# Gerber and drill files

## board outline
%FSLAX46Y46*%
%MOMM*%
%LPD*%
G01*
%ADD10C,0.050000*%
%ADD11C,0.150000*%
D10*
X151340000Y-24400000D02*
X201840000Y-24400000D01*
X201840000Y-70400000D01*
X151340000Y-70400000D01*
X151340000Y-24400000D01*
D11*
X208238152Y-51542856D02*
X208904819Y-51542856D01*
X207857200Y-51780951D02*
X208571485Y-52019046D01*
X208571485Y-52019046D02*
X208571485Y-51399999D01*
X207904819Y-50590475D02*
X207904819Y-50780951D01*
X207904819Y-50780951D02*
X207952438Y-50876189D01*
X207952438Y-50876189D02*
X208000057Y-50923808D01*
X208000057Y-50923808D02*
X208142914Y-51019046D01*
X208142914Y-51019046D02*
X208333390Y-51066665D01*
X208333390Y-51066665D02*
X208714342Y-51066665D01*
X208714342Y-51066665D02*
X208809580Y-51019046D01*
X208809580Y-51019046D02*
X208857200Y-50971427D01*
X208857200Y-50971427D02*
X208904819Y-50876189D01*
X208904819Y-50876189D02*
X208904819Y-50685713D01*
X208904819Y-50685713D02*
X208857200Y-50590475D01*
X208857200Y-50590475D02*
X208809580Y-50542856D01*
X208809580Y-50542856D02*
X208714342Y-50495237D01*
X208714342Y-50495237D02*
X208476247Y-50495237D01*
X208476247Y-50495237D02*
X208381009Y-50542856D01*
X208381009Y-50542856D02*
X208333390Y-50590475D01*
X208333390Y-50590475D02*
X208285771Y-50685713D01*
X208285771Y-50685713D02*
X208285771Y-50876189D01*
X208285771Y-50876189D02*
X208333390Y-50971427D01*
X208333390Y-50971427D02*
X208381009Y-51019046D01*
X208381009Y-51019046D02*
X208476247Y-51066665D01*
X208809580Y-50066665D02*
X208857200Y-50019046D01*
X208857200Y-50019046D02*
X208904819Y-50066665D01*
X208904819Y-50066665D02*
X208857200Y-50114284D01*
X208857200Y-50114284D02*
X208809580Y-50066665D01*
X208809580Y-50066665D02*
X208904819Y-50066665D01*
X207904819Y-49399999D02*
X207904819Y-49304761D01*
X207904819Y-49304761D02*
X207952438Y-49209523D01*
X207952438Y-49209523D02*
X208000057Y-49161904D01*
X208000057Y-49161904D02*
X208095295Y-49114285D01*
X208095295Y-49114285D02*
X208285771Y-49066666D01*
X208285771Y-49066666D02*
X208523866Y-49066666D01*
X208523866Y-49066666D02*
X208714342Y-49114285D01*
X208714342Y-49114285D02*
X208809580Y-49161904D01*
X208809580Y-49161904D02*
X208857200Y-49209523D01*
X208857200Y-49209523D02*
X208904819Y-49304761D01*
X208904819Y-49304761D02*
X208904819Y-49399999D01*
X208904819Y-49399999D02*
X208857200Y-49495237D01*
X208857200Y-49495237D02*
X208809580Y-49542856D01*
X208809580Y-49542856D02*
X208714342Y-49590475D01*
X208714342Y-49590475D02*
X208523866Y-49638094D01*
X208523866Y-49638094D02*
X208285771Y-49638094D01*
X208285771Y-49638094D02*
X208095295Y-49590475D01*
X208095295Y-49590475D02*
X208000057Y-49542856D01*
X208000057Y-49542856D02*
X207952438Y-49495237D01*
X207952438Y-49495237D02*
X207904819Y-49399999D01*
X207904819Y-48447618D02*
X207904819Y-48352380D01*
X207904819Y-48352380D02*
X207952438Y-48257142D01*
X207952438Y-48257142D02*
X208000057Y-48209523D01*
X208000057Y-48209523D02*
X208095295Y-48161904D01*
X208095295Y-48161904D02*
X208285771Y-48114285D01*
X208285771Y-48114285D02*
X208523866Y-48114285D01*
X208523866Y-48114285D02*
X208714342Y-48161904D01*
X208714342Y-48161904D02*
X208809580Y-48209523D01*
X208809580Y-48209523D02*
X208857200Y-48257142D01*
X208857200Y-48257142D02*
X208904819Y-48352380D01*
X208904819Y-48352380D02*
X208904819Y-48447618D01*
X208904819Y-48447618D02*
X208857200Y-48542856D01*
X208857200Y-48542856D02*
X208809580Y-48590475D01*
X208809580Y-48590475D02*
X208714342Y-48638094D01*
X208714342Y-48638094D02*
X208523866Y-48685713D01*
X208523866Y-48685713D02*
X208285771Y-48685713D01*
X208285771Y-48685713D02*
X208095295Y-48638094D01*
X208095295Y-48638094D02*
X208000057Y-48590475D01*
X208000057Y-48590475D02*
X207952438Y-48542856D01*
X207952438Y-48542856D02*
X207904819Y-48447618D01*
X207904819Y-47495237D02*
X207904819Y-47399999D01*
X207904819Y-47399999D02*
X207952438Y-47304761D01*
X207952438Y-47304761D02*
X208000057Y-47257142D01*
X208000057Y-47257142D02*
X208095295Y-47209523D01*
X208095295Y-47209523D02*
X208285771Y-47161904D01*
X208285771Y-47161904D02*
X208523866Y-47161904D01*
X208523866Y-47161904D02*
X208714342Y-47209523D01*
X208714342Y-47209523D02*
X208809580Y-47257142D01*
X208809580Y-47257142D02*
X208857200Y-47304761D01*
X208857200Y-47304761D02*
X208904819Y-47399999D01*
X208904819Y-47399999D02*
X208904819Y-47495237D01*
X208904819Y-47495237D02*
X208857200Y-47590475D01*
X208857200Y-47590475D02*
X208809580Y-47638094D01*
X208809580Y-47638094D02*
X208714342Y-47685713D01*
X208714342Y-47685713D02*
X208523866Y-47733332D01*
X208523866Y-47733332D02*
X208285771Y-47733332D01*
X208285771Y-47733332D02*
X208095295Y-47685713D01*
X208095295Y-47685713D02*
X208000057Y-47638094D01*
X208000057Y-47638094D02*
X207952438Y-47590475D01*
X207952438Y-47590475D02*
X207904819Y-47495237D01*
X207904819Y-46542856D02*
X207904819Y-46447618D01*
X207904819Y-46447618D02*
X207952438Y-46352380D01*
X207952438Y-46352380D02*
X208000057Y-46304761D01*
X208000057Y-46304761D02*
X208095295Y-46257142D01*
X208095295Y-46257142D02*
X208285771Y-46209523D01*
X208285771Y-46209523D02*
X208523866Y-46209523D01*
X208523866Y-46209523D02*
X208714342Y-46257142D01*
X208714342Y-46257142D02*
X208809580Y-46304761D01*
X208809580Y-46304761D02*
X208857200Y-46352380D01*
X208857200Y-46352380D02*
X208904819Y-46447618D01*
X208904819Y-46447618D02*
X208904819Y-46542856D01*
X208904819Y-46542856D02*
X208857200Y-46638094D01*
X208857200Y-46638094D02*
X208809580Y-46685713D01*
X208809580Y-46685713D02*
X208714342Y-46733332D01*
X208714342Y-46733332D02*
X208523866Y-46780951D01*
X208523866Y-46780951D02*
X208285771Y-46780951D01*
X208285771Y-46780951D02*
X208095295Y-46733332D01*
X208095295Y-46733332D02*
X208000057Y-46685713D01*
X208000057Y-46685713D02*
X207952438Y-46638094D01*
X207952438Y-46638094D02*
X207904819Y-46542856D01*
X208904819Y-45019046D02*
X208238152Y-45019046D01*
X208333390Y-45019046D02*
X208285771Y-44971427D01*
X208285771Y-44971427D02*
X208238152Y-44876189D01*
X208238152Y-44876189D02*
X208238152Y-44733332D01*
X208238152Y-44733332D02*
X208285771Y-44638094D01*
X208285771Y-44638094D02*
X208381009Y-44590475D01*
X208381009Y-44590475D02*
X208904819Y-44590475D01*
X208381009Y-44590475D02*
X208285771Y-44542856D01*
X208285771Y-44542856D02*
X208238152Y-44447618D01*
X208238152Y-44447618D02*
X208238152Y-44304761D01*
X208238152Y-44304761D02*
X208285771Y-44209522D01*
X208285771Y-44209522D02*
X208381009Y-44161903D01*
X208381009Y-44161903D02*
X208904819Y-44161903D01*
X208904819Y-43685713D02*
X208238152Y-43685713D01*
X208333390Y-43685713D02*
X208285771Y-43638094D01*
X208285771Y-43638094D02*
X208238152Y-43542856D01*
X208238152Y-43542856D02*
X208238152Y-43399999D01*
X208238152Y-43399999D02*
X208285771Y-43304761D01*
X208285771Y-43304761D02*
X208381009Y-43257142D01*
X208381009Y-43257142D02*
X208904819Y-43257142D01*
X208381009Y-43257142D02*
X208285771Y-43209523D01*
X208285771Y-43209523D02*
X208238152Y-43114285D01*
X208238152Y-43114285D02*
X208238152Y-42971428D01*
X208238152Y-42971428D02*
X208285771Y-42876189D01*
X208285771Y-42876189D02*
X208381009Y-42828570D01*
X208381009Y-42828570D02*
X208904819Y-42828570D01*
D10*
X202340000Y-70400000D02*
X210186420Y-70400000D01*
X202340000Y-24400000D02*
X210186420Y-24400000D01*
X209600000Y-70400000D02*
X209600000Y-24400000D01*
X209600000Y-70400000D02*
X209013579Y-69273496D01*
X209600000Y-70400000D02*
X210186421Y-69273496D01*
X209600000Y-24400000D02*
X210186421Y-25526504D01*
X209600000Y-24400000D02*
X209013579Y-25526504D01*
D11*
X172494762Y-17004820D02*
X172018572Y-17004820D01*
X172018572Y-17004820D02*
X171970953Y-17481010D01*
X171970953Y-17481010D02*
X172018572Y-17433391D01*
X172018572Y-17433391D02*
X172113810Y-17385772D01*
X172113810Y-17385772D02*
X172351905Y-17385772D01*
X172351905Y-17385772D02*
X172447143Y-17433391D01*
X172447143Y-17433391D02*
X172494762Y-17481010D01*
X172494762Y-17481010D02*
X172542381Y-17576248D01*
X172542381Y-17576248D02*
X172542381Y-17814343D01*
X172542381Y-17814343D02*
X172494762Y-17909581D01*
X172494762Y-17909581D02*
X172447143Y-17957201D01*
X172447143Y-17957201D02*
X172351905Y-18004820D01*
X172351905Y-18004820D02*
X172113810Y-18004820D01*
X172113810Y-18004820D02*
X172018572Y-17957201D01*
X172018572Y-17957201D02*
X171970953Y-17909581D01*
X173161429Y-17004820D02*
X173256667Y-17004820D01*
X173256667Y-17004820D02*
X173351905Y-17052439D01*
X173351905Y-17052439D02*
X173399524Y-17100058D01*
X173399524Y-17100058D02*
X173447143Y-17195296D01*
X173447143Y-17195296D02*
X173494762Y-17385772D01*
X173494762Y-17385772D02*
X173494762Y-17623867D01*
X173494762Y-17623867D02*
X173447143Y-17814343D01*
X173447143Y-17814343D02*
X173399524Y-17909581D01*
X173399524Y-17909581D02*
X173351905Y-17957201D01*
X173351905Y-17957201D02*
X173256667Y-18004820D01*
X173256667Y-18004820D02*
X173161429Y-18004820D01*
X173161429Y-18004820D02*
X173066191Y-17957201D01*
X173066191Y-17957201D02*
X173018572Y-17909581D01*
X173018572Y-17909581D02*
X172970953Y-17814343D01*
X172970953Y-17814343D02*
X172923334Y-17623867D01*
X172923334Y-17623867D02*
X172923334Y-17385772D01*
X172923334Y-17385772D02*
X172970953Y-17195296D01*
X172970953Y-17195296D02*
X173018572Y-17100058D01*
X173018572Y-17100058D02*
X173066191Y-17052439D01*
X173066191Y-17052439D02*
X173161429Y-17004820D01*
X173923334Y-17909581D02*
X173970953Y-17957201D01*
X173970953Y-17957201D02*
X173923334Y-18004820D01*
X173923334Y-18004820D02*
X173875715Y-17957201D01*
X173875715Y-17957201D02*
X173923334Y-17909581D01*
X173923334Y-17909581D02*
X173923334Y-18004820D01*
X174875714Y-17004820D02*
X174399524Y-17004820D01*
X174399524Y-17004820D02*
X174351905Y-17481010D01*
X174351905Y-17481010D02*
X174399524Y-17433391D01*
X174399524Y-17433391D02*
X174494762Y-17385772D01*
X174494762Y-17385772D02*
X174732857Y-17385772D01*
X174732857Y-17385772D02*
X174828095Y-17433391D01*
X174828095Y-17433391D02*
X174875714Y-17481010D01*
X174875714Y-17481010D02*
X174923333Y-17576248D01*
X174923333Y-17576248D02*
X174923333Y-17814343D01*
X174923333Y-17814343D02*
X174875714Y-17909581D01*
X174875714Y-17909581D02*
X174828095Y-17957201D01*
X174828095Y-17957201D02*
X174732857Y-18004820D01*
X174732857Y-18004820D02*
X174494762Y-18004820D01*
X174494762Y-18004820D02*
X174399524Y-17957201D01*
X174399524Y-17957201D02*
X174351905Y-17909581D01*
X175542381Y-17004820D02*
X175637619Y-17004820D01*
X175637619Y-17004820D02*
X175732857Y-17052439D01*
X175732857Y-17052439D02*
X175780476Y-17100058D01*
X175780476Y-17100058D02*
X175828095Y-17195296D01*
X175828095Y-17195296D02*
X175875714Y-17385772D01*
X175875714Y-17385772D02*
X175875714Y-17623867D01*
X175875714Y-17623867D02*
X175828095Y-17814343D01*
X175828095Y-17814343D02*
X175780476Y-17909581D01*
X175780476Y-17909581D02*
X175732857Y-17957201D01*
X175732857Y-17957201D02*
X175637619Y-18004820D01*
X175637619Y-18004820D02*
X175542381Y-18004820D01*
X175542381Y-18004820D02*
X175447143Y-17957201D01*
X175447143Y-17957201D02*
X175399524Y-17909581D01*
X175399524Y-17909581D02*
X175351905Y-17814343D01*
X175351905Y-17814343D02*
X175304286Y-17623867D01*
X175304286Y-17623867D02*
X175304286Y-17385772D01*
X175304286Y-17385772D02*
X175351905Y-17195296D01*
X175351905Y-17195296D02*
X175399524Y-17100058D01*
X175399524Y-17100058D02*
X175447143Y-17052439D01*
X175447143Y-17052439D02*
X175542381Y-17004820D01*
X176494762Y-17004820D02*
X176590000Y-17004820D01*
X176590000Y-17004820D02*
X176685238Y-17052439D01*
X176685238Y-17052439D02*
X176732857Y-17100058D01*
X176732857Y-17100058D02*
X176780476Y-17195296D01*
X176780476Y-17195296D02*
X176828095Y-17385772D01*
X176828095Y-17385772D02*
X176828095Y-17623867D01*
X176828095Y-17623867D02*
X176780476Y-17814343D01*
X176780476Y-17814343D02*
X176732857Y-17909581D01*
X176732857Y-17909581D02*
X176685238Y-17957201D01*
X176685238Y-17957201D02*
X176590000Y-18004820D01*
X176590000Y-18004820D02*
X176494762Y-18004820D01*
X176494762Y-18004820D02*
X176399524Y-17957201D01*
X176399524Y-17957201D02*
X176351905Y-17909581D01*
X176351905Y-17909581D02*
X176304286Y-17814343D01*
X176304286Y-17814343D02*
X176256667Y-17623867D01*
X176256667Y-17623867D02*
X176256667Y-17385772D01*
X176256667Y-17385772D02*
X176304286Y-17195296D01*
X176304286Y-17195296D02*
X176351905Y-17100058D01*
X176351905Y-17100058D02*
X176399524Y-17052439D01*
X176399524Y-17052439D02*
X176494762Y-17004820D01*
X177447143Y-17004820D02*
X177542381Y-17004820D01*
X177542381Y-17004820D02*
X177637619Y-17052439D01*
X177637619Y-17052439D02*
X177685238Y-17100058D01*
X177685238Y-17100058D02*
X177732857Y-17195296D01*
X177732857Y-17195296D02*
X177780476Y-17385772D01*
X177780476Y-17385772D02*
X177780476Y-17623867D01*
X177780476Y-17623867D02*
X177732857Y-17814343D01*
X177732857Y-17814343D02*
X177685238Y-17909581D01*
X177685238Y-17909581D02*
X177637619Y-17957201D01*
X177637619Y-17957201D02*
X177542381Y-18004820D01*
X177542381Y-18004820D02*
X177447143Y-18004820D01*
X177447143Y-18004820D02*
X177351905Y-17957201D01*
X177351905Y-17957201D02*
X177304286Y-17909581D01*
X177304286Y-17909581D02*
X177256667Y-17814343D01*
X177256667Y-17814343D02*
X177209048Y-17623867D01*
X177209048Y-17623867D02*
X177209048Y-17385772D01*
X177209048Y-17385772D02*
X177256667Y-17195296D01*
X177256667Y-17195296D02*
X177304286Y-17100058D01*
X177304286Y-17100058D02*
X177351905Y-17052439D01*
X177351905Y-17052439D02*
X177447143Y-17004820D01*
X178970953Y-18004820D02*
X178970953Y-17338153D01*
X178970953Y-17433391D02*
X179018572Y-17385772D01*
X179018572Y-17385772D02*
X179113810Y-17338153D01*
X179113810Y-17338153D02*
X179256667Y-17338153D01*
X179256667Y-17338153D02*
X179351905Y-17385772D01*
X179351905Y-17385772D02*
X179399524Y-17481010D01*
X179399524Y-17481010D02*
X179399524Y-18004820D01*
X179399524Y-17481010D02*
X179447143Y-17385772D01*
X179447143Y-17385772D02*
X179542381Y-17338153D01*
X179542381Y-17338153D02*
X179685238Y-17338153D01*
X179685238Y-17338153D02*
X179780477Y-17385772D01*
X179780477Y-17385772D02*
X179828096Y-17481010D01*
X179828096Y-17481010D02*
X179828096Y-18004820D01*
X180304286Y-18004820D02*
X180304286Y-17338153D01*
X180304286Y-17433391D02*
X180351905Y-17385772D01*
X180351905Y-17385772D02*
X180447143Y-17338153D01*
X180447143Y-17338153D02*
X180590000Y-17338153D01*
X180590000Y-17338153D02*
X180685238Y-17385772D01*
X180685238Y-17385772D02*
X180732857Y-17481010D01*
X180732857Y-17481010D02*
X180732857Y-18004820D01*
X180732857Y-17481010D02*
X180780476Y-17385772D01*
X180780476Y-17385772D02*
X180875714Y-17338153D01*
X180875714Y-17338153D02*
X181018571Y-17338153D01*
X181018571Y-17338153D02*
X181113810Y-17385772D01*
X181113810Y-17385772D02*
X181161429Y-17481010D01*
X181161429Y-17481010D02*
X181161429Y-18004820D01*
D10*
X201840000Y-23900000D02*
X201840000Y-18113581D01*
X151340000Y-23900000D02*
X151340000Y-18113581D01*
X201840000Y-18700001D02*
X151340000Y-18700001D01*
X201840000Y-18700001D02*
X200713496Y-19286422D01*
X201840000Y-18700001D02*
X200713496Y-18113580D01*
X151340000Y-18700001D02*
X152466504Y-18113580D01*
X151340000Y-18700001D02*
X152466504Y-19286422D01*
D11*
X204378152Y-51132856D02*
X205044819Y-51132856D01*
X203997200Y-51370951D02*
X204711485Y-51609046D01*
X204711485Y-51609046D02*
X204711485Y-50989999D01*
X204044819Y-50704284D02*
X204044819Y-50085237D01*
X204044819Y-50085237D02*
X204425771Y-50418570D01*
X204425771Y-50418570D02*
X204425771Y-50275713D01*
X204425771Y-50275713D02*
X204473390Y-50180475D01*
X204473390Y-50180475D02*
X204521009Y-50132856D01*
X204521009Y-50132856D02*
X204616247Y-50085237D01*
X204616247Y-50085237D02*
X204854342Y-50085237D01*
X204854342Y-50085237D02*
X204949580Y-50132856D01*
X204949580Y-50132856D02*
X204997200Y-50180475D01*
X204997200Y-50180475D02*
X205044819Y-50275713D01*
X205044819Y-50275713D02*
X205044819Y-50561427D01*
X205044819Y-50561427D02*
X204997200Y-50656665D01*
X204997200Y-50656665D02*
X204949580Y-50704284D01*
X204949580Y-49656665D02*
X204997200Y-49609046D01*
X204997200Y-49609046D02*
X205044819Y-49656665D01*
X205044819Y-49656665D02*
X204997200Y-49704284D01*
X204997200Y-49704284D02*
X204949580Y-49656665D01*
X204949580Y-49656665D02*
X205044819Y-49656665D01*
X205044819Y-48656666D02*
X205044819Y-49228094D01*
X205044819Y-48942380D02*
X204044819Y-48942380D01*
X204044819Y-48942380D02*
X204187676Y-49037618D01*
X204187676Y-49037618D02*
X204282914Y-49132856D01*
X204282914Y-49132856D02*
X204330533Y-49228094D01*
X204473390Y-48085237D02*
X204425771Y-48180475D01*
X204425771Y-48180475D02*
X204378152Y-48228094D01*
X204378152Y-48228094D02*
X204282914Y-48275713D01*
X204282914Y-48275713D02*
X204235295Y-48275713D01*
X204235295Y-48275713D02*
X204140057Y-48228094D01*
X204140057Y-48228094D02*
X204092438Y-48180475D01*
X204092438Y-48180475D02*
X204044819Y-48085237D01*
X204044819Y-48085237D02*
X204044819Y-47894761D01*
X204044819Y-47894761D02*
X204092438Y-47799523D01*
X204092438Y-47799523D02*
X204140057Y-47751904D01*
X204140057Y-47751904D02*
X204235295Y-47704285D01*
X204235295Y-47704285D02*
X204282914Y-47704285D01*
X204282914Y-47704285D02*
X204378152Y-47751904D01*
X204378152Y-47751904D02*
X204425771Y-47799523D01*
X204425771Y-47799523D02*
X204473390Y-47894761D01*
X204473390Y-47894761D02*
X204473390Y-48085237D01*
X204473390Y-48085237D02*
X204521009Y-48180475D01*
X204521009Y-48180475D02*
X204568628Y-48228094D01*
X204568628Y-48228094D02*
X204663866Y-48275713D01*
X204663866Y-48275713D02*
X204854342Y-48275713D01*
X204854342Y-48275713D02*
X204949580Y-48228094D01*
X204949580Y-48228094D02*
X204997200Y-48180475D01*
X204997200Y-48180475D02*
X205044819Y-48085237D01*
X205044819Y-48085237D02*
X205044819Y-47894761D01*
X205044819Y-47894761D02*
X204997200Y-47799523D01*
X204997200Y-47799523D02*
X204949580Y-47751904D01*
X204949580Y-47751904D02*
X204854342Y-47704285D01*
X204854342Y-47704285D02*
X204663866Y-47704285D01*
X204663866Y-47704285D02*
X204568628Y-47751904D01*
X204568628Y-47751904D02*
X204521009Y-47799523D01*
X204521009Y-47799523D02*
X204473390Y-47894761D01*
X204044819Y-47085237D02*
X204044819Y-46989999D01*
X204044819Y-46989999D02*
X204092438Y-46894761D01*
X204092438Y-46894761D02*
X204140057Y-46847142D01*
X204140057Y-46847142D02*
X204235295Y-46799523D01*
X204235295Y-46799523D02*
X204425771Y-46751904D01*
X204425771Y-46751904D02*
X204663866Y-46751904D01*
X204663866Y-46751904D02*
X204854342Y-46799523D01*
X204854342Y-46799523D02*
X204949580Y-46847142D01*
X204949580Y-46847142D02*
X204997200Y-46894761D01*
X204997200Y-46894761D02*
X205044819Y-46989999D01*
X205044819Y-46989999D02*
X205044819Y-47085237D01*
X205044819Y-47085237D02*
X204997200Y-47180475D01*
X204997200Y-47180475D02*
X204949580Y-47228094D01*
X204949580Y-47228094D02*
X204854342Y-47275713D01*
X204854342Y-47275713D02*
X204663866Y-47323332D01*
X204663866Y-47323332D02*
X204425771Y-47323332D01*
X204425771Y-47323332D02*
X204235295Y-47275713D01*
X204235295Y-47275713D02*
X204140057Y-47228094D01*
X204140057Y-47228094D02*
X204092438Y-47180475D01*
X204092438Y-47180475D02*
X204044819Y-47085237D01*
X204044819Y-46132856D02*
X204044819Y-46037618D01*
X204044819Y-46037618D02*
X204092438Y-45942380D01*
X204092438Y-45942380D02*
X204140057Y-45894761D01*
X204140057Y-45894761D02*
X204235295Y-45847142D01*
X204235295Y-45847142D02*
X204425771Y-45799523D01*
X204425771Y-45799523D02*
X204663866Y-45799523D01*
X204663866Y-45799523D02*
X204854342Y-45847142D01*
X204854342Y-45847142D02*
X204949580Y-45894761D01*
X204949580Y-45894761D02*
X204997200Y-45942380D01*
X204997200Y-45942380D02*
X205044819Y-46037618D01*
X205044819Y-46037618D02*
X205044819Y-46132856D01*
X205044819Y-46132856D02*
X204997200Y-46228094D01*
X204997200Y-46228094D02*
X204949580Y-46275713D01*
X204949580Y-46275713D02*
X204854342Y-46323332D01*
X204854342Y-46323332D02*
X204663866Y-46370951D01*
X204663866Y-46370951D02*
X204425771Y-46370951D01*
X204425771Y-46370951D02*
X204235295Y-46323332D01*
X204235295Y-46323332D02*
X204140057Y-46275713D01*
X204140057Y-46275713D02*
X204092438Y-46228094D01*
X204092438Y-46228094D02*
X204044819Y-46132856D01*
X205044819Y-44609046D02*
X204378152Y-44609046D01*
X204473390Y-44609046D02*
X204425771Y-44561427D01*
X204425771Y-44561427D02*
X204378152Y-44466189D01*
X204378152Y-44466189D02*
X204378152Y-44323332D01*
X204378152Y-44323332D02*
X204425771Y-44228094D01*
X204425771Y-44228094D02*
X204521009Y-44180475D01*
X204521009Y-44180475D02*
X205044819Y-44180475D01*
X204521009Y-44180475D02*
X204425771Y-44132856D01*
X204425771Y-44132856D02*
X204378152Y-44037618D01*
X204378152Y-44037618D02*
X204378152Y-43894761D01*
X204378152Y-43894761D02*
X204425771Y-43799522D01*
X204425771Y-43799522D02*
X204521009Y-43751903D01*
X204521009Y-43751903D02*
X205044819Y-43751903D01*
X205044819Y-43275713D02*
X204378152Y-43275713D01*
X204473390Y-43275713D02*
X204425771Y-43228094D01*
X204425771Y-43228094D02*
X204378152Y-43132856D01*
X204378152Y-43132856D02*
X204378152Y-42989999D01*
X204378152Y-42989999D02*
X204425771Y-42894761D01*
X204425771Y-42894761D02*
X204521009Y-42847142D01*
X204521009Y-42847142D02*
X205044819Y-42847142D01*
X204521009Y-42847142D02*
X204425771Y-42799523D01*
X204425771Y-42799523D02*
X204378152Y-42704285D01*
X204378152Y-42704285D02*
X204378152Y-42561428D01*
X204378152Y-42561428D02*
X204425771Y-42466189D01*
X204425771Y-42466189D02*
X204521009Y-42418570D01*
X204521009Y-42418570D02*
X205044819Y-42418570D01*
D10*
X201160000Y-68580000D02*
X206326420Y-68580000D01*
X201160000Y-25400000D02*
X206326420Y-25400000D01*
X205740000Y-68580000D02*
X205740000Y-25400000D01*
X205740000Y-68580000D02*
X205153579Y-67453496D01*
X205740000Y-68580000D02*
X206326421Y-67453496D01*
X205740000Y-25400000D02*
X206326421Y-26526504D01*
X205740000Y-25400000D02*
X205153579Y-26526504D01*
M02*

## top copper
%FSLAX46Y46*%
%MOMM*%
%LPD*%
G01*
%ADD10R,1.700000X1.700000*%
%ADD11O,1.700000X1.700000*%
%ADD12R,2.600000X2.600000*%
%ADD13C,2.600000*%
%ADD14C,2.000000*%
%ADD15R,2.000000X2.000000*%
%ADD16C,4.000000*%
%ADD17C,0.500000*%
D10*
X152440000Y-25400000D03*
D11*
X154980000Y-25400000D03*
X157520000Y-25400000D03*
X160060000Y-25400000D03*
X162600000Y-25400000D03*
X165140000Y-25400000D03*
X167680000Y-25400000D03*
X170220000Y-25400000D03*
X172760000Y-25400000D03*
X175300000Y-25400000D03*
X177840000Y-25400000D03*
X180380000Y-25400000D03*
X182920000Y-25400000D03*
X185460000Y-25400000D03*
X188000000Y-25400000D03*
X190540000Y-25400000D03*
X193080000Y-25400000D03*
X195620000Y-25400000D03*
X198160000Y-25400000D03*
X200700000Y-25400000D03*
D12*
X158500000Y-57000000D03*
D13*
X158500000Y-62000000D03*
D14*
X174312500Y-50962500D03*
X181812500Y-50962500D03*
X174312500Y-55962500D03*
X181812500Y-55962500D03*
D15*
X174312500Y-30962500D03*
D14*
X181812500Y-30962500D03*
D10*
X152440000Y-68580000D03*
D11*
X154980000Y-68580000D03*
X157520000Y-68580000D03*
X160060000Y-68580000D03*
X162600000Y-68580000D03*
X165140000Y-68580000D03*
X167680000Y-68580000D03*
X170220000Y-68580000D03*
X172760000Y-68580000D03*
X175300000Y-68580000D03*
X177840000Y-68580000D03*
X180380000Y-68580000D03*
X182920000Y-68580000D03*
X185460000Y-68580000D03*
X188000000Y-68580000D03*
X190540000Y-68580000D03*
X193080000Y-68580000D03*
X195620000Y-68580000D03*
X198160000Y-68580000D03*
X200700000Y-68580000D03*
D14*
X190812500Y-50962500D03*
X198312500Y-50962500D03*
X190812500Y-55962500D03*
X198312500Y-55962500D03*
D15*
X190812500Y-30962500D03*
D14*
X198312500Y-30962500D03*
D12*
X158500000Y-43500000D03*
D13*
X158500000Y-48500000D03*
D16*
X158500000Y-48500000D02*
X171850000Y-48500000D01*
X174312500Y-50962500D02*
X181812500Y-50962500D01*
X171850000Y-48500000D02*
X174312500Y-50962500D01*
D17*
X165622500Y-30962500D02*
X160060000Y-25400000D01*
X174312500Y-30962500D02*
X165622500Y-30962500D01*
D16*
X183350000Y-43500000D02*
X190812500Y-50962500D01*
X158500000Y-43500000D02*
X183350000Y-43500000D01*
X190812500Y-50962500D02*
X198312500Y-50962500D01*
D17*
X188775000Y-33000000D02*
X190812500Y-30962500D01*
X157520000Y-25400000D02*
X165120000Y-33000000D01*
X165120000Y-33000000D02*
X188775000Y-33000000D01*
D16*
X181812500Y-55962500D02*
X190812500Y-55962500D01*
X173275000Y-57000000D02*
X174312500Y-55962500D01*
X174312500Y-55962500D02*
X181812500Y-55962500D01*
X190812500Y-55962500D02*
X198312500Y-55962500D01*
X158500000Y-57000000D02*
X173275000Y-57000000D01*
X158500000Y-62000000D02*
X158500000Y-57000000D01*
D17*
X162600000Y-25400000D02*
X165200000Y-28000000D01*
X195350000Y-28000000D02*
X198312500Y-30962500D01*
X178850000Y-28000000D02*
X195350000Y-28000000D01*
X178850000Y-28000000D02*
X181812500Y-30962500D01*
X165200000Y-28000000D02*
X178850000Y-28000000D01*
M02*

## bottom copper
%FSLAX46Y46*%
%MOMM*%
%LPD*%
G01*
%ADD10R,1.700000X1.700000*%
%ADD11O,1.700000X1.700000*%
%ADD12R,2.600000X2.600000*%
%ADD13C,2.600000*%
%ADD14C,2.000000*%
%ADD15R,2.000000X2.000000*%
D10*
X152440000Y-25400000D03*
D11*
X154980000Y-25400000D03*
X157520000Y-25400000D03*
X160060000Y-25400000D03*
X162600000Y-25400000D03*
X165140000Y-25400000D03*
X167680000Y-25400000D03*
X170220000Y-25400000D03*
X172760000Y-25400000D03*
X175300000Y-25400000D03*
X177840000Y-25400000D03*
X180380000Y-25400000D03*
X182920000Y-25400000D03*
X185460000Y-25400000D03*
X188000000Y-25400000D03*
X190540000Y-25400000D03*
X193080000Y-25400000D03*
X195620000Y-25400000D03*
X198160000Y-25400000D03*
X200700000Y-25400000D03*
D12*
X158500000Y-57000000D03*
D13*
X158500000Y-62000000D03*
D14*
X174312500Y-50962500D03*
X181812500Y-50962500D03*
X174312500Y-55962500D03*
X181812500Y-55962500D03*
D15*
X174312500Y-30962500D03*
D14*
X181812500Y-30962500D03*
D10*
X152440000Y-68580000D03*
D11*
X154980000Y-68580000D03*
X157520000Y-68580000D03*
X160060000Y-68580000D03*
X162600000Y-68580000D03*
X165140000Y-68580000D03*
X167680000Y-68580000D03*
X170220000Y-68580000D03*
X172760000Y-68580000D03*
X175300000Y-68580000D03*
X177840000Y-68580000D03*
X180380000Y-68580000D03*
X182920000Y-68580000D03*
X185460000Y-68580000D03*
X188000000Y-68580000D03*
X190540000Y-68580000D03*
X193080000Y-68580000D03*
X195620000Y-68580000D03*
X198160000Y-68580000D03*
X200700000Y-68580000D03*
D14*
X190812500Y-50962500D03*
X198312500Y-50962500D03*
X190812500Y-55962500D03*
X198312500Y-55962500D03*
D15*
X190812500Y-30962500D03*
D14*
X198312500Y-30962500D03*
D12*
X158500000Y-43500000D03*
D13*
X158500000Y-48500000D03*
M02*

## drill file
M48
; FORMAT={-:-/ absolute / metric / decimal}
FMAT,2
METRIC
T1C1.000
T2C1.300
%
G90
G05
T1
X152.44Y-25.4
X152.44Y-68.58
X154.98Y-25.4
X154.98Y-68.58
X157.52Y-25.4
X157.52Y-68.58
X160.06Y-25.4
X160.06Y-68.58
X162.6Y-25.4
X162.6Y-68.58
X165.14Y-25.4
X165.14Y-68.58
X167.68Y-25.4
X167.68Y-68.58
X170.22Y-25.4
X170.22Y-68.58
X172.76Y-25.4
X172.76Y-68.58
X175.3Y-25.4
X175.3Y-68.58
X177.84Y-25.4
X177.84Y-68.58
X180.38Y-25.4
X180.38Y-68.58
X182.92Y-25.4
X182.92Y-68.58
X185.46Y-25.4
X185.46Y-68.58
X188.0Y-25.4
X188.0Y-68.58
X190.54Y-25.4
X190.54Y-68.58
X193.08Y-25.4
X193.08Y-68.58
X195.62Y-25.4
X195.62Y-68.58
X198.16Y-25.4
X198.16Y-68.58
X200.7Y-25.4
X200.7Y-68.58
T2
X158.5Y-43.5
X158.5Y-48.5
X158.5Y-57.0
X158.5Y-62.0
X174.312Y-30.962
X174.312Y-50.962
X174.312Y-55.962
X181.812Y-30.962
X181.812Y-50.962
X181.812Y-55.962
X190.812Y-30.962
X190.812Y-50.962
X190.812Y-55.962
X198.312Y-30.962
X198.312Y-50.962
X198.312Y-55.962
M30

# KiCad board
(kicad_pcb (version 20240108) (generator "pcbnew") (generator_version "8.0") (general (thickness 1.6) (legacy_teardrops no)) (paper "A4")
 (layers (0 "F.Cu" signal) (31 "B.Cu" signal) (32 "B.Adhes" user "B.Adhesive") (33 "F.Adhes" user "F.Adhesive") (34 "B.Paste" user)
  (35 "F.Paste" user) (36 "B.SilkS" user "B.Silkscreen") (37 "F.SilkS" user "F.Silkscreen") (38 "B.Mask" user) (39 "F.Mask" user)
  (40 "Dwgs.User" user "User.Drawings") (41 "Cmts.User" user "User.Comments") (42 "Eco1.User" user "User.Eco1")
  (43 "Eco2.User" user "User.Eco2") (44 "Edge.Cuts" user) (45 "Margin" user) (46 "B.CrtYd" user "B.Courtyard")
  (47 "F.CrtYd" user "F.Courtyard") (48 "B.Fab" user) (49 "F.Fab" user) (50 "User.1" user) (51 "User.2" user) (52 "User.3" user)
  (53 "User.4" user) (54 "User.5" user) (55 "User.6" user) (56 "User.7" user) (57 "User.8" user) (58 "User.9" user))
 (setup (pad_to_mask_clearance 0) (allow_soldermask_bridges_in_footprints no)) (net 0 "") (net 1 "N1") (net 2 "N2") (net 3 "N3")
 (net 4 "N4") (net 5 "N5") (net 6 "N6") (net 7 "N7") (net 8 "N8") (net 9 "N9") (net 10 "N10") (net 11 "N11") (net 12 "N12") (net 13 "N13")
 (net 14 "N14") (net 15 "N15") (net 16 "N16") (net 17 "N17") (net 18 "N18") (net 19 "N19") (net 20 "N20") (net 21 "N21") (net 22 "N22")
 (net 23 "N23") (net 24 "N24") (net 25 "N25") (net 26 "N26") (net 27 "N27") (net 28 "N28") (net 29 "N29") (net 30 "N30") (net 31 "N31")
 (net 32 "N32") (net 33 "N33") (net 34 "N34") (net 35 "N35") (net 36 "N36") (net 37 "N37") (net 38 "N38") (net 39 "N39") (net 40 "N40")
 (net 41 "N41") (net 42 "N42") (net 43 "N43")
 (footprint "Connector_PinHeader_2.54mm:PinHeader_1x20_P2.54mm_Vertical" (layer "F.Cu") (at 152.44 25.4 90)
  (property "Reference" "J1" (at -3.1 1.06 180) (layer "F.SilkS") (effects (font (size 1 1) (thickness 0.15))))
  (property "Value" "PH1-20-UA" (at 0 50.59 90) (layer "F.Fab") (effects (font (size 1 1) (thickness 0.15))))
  (pad "1" thru_hole rect (at 0 0 90) (size 1.7 1.7) (drill 1) (layers "*.Cu" "*.Mask") (remove_unused_layers no) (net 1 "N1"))
  (pad "2" thru_hole oval (at 0 2.54 90) (size 1.7 1.7) (drill 1) (layers "*.Cu" "*.Mask") (remove_unused_layers no) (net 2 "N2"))
  (pad "3" thru_hole oval (at 0 5.08 90) (size 1.7 1.7) (drill 1) (layers "*.Cu" "*.Mask") (remove_unused_layers no) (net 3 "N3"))
  (pad "4" thru_hole oval (at 0 7.62 90) (size 1.7 1.7) (drill 1) (layers "*.Cu" "*.Mask") (remove_unused_layers no) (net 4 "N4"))
  (pad "5" thru_hole oval (at 0 10.16 90) (size 1.7 1.7) (drill 1) (layers "*.Cu" "*.Mask") (remove_unused_layers no) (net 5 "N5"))
  (pad "6" thru_hole oval (at 0 12.7 90) (size 1.7 1.7) (drill 1) (layers "*.Cu" "*.Mask") (remove_unused_layers no) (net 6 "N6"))
  (pad "7" thru_hole oval (at 0 15.24 90) (size 1.7 1.7) (drill 1) (layers "*.Cu" "*.Mask") (remove_unused_layers no) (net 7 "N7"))
  (pad "8" thru_hole oval (at 0 17.78 90) (size 1.7 1.7) (drill 1) (layers "*.Cu" "*.Mask") (remove_unused_layers no) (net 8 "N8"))
  (pad "9" thru_hole oval (at 0 20.32 90) (size 1.7 1.7) (drill 1) (layers "*.Cu" "*.Mask") (remove_unused_layers no) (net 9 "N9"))
  (pad "10" thru_hole oval (at 0 22.86 90) (size 1.7 1.7) (drill 1) (layers "*.Cu" "*.Mask") (remove_unused_layers no) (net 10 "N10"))
  (pad "11" thru_hole oval (at 0 25.4 90) (size 1.7 1.7) (drill 1) (layers "*.Cu" "*.Mask") (remove_unused_layers no) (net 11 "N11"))
  (pad "12" thru_hole oval (at 0 27.94 90) (size 1.7 1.7) (drill 1) (layers "*.Cu" "*.Mask") (remove_unused_layers no) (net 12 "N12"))
  (pad "13" thru_hole oval (at 0 30.48 90) (size 1.7 1.7) (drill 1) (layers "*.Cu" "*.Mask") (remove_unused_layers no) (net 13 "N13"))
  (pad "14" thru_hole oval (at 0 33.02 90) (size 1.7 1.7) (drill 1) (layers "*.Cu" "*.Mask") (remove_unused_layers no) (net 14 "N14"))
  (pad "15" thru_hole oval (at 0 35.56 90) (size 1.7 1.7) (drill 1) (layers "*.Cu" "*.Mask") (remove_unused_layers no) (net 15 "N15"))
  (pad "16" thru_hole oval (at 0 38.1 90) (size 1.7 1.7) (drill 1) (layers "*.Cu" "*.Mask") (remove_unused_layers no) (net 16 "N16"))
  (pad "17" thru_hole oval (at 0 40.64 90) (size 1.7 1.7) (drill 1) (layers "*.Cu" "*.Mask") (remove_unused_layers no) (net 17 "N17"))
  (pad "18" thru_hole oval (at 0 43.18 90) (size 1.7 1.7) (drill 1) (layers "*.Cu" "*.Mask") (remove_unused_layers no) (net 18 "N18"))
  (pad "19" thru_hole oval (at 0 45.72 90) (size 1.7 1.7) (drill 1) (layers "*.Cu" "*.Mask") (remove_unused_layers no) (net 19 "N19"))
  (pad "20" thru_hole oval (at 0 48.26 90) (size 1.7 1.7) (drill 1) (layers "*.Cu" "*.Mask") (remove_unused_layers no) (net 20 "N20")))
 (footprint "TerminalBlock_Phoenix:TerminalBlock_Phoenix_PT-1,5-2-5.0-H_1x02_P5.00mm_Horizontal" (layer "F.Cu") (at 158.5 57 -90)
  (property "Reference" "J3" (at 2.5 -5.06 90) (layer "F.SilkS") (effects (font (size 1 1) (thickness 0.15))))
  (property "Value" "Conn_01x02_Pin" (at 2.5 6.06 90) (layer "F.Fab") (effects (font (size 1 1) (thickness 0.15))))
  (pad "1" thru_hole rect (at 0 0 270) (size 2.6 2.6) (drill 1.3) (layers "*.Cu" "*.Mask") (remove_unused_layers no) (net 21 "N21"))
  (pad "2" thru_hole circle (at 5 0 270) (size 2.6 2.6) (drill 1.3) (layers "*.Cu" "*.Mask") (remove_unused_layers no) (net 21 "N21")))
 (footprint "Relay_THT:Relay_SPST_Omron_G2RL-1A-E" (layer "F.Cu") (at 174.3125 30.9625)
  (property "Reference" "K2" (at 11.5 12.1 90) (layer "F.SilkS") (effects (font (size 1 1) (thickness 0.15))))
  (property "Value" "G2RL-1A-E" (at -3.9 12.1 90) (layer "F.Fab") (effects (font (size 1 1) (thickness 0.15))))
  (pad "13" thru_hole circle (at 0 20) (size 2 2) (drill 1.3) (layers "*.Cu" "*.Mask") (remove_unused_layers no) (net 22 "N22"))
  (pad "13" thru_hole circle (at 7.5 20) (size 2 2) (drill 1.3) (layers "*.Cu" "*.Mask") (remove_unused_layers no) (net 22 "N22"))
  (pad "14" thru_hole circle (at 0 25) (size 2 2) (drill 1.3) (layers "*.Cu" "*.Mask") (remove_unused_layers no) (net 21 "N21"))
  (pad "14" thru_hole circle (at 7.5 25) (size 2 2) (drill 1.3) (layers "*.Cu" "*.Mask") (remove_unused_layers no) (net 21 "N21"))
  (pad "A1" thru_hole rect (at 0 0) (size 2 2) (drill 1.3) (layers "*.Cu" "*.Mask") (remove_unused_layers no) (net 4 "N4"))
  (pad "A2" thru_hole circle (at 7.5 0) (size 2 2) (drill 1.3) (layers "*.Cu" "*.Mask") (remove_unused_layers no) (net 5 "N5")))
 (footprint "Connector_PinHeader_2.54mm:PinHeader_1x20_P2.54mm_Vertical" (layer "F.Cu") (at 152.44 68.58 90)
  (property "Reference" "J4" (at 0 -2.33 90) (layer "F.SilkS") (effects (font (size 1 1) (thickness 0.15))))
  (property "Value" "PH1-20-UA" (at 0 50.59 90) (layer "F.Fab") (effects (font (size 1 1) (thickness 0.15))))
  (pad "1" thru_hole rect (at 0 0 90) (size 1.7 1.7) (drill 1) (layers "*.Cu" "*.Mask") (remove_unused_layers no) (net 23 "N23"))
  (pad "2" thru_hole oval (at 0 2.54 90) (size 1.7 1.7) (drill 1) (layers "*.Cu" "*.Mask") (remove_unused_layers no) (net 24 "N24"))
  (pad "3" thru_hole oval (at 0 5.08 90) (size 1.7 1.7) (drill 1) (layers "*.Cu" "*.Mask") (remove_unused_layers no) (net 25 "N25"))
  (pad "4" thru_hole oval (at 0 7.62 90) (size 1.7 1.7) (drill 1) (layers "*.Cu" "*.Mask") (remove_unused_layers no) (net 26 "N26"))
  (pad "5" thru_hole oval (at 0 10.16 90) (size 1.7 1.7) (drill 1) (layers "*.Cu" "*.Mask") (remove_unused_layers no) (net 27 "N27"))
  (pad "6" thru_hole oval (at 0 12.7 90) (size 1.7 1.7) (drill 1) (layers "*.Cu" "*.Mask") (remove_unused_layers no) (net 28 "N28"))
  (pad "7" thru_hole oval (at 0 15.24 90) (size 1.7 1.7) (drill 1) (layers "*.Cu" "*.Mask") (remove_unused_layers no) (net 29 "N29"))
  (pad "8" thru_hole oval (at 0 17.78 90) (size 1.7 1.7) (drill 1) (layers "*.Cu" "*.Mask") (remove_unused_layers no) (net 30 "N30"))
  (pad "9" thru_hole oval (at 0 20.32 90) (size 1.7 1.7) (drill 1) (layers "*.Cu" "*.Mask") (remove_unused_layers no) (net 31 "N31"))
  (pad "10" thru_hole oval (at 0 22.86 90) (size 1.7 1.7) (drill 1) (layers "*.Cu" "*.Mask") (remove_unused_layers no) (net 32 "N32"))
  (pad "11" thru_hole oval (at 0 25.4 90) (size 1.7 1.7) (drill 1) (layers "*.Cu" "*.Mask") (remove_unused_layers no) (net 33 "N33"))
  (pad "12" thru_hole oval (at 0 27.94 90) (size 1.7 1.7) (drill 1) (layers "*.Cu" "*.Mask") (remove_unused_layers no) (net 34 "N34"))
  (pad "13" thru_hole oval (at 0 30.48 90) (size 1.7 1.7) (drill 1) (layers "*.Cu" "*.Mask") (remove_unused_layers no) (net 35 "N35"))
  (pad "14" thru_hole oval (at 0 33.02 90) (size 1.7 1.7) (drill 1) (layers "*.Cu" "*.Mask") (remove_unused_layers no) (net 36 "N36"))
  (pad "15" thru_hole oval (at 0 35.56 90) (size 1.7 1.7) (drill 1) (layers "*.Cu" "*.Mask") (remove_unused_layers no) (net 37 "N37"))
  (pad "16" thru_hole oval (at 0 38.1 90) (size 1.7 1.7) (drill 1) (layers "*.Cu" "*.Mask") (remove_unused_layers no) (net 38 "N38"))
  (pad "17" thru_hole oval (at 0 40.64 90) (size 1.7 1.7) (drill 1) (layers "*.Cu" "*.Mask") (remove_unused_layers no) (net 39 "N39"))
  (pad "18" thru_hole oval (at 0 43.18 90) (size 1.7 1.7) (drill 1) (layers "*.Cu" "*.Mask") (remove_unused_layers no) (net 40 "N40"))
  (pad "19" thru_hole oval (at 0 45.72 90) (size 1.7 1.7) (drill 1) (layers "*.Cu" "*.Mask") (remove_unused_layers no) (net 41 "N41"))
  (pad "20" thru_hole oval (at 0 48.26 90) (size 1.7 1.7) (drill 1) (layers "*.Cu" "*.Mask") (remove_unused_layers no) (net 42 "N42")))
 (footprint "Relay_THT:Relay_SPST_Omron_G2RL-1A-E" (layer "F.Cu") (at 190.8125 30.9625)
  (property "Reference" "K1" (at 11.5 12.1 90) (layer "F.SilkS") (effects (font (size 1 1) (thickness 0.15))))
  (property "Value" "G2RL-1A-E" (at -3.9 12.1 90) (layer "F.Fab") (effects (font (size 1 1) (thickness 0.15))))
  (pad "13" thru_hole circle (at 0 20) (size 2 2) (drill 1.3) (layers "*.Cu" "*.Mask") (remove_unused_layers no) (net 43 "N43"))
  (pad "13" thru_hole circle (at 7.5 20) (size 2 2) (drill 1.3) (layers "*.Cu" "*.Mask") (remove_unused_layers no) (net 43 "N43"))
  (pad "14" thru_hole circle (at 0 25) (size 2 2) (drill 1.3) (layers "*.Cu" "*.Mask") (remove_unused_layers no) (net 21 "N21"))
  (pad "14" thru_hole circle (at 7.5 25) (size 2 2) (drill 1.3) (layers "*.Cu" "*.Mask") (remove_unused_layers no) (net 21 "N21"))
  (pad "A1" thru_hole rect (at 0 0) (size 2 2) (drill 1.3) (layers "*.Cu" "*.Mask") (remove_unused_layers no) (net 3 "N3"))
  (pad "A2" thru_hole circle (at 7.5 0) (size 2 2) (drill 1.3) (layers "*.Cu" "*.Mask") (remove_unused_layers no) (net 5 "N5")))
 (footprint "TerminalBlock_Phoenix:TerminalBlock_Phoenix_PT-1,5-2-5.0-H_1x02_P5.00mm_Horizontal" (layer "F.Cu") (at 158.5 43.5 -90)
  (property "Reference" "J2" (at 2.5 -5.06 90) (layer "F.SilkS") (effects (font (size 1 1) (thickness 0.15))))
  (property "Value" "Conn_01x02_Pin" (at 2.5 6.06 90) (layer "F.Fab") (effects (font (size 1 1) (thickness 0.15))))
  (pad "1" thru_hole rect (at 0 0 270) (size 2.6 2.6) (drill 1.3) (layers "*.Cu" "*.Mask") (remove_unused_layers no) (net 43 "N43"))
  (pad "2" thru_hole circle (at 5 0 270) (size 2.6 2.6) (drill 1.3) (layers "*.Cu" "*.Mask") (remove_unused_layers no) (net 22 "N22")))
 (gr_rect (start 151.34 24.4) (end 201.84 70.4) (stroke (width 0.05) (type default)) (fill none) (layer "Edge.Cuts"))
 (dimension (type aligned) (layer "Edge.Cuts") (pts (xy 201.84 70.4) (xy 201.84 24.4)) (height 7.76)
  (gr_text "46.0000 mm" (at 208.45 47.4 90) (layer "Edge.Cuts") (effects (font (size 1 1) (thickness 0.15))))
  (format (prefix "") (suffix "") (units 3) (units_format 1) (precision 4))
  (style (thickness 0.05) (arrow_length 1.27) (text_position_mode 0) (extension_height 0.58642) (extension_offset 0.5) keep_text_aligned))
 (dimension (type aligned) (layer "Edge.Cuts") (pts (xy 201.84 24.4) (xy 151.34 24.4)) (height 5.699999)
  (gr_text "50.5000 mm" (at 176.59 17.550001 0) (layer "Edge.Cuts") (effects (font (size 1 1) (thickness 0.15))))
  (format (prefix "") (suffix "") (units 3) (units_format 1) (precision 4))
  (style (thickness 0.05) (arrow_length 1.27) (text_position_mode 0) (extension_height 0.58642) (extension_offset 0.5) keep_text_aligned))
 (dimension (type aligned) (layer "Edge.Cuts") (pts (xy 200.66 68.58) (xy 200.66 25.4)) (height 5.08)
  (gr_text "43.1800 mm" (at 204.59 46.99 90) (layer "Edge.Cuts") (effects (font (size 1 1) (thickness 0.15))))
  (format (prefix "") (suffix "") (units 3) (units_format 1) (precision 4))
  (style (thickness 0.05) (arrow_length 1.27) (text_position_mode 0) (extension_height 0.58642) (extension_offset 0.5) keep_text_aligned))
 (segment (start 158.5 48.5) (end 171.85 48.5) (width 4) (layer "F.Cu") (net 22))
 (segment (start 174.3125 50.9625) (end 181.8125 50.9625) (width 4) (layer "F.Cu") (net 22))
 (segment (start 171.85 48.5) (end 174.3125 50.9625) (width 4) (layer "F.Cu") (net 22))
 (segment (start 165.6225 30.9625) (end 160.06 25.4) (width 0.5) (layer "F.Cu") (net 4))
 (segment (start 174.3125 30.9625) (end 165.6225 30.9625) (width 0.5) (layer "F.Cu") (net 4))
 (segment (start 183.35 43.5) (end 190.8125 50.9625) (width 4) (layer "F.Cu") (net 43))
 (segment (start 158.5 43.5) (end 183.35 43.5) (width 4) (layer "F.Cu") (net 43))
 (segment (start 190.8125 50.9625) (end 198.3125 50.9625) (width 4) (layer "F.Cu") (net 43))
 (segment (start 188.775 33) (end 190.8125 30.9625) (width 0.5) (layer "F.Cu") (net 3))
 (segment (start 157.52 25.4) (end 165.12 33) (width 0.5) (layer "F.Cu") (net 3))
 (segment (start 165.12 33) (end 188.775 33) (width 0.5) (layer "F.Cu") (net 3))
 (segment (start 181.8125 55.9625) (end 190.8125 55.9625) (width 4) (layer "F.Cu") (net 21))
 (segment (start 173.275 57) (end 174.3125 55.9625) (width 4) (layer "F.Cu") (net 21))
 (segment (start 174.3125 55.9625) (end 181.8125 55.9625) (width 4) (layer "F.Cu") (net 21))
 (segment (start 190.8125 55.9625) (end 198.3125 55.9625) (width 4) (layer "F.Cu") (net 21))
 (segment (start 158.5 57) (end 173.275 57) (width 4) (layer "F.Cu") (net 21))
 (segment (start 158.5 62) (end 158.5 57) (width 4) (layer "F.Cu") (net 21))
 (segment (start 162.6 25.4) (end 165.2 28) (width 0.5) (layer "F.Cu") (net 5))
 (segment (start 195.35 28) (end 198.3125 30.9625) (width 0.5) (layer "F.Cu") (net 5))
 (segment (start 178.85 28) (end 195.35 28) (width 0.5) (layer "F.Cu") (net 5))
 (segment (start 178.85 28) (end 181.8125 30.9625) (width 0.5) (layer "F.Cu") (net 5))
 (segment (start 165.2 28) (end 178.85 28) (width 0.5) (layer "F.Cu") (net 5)))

